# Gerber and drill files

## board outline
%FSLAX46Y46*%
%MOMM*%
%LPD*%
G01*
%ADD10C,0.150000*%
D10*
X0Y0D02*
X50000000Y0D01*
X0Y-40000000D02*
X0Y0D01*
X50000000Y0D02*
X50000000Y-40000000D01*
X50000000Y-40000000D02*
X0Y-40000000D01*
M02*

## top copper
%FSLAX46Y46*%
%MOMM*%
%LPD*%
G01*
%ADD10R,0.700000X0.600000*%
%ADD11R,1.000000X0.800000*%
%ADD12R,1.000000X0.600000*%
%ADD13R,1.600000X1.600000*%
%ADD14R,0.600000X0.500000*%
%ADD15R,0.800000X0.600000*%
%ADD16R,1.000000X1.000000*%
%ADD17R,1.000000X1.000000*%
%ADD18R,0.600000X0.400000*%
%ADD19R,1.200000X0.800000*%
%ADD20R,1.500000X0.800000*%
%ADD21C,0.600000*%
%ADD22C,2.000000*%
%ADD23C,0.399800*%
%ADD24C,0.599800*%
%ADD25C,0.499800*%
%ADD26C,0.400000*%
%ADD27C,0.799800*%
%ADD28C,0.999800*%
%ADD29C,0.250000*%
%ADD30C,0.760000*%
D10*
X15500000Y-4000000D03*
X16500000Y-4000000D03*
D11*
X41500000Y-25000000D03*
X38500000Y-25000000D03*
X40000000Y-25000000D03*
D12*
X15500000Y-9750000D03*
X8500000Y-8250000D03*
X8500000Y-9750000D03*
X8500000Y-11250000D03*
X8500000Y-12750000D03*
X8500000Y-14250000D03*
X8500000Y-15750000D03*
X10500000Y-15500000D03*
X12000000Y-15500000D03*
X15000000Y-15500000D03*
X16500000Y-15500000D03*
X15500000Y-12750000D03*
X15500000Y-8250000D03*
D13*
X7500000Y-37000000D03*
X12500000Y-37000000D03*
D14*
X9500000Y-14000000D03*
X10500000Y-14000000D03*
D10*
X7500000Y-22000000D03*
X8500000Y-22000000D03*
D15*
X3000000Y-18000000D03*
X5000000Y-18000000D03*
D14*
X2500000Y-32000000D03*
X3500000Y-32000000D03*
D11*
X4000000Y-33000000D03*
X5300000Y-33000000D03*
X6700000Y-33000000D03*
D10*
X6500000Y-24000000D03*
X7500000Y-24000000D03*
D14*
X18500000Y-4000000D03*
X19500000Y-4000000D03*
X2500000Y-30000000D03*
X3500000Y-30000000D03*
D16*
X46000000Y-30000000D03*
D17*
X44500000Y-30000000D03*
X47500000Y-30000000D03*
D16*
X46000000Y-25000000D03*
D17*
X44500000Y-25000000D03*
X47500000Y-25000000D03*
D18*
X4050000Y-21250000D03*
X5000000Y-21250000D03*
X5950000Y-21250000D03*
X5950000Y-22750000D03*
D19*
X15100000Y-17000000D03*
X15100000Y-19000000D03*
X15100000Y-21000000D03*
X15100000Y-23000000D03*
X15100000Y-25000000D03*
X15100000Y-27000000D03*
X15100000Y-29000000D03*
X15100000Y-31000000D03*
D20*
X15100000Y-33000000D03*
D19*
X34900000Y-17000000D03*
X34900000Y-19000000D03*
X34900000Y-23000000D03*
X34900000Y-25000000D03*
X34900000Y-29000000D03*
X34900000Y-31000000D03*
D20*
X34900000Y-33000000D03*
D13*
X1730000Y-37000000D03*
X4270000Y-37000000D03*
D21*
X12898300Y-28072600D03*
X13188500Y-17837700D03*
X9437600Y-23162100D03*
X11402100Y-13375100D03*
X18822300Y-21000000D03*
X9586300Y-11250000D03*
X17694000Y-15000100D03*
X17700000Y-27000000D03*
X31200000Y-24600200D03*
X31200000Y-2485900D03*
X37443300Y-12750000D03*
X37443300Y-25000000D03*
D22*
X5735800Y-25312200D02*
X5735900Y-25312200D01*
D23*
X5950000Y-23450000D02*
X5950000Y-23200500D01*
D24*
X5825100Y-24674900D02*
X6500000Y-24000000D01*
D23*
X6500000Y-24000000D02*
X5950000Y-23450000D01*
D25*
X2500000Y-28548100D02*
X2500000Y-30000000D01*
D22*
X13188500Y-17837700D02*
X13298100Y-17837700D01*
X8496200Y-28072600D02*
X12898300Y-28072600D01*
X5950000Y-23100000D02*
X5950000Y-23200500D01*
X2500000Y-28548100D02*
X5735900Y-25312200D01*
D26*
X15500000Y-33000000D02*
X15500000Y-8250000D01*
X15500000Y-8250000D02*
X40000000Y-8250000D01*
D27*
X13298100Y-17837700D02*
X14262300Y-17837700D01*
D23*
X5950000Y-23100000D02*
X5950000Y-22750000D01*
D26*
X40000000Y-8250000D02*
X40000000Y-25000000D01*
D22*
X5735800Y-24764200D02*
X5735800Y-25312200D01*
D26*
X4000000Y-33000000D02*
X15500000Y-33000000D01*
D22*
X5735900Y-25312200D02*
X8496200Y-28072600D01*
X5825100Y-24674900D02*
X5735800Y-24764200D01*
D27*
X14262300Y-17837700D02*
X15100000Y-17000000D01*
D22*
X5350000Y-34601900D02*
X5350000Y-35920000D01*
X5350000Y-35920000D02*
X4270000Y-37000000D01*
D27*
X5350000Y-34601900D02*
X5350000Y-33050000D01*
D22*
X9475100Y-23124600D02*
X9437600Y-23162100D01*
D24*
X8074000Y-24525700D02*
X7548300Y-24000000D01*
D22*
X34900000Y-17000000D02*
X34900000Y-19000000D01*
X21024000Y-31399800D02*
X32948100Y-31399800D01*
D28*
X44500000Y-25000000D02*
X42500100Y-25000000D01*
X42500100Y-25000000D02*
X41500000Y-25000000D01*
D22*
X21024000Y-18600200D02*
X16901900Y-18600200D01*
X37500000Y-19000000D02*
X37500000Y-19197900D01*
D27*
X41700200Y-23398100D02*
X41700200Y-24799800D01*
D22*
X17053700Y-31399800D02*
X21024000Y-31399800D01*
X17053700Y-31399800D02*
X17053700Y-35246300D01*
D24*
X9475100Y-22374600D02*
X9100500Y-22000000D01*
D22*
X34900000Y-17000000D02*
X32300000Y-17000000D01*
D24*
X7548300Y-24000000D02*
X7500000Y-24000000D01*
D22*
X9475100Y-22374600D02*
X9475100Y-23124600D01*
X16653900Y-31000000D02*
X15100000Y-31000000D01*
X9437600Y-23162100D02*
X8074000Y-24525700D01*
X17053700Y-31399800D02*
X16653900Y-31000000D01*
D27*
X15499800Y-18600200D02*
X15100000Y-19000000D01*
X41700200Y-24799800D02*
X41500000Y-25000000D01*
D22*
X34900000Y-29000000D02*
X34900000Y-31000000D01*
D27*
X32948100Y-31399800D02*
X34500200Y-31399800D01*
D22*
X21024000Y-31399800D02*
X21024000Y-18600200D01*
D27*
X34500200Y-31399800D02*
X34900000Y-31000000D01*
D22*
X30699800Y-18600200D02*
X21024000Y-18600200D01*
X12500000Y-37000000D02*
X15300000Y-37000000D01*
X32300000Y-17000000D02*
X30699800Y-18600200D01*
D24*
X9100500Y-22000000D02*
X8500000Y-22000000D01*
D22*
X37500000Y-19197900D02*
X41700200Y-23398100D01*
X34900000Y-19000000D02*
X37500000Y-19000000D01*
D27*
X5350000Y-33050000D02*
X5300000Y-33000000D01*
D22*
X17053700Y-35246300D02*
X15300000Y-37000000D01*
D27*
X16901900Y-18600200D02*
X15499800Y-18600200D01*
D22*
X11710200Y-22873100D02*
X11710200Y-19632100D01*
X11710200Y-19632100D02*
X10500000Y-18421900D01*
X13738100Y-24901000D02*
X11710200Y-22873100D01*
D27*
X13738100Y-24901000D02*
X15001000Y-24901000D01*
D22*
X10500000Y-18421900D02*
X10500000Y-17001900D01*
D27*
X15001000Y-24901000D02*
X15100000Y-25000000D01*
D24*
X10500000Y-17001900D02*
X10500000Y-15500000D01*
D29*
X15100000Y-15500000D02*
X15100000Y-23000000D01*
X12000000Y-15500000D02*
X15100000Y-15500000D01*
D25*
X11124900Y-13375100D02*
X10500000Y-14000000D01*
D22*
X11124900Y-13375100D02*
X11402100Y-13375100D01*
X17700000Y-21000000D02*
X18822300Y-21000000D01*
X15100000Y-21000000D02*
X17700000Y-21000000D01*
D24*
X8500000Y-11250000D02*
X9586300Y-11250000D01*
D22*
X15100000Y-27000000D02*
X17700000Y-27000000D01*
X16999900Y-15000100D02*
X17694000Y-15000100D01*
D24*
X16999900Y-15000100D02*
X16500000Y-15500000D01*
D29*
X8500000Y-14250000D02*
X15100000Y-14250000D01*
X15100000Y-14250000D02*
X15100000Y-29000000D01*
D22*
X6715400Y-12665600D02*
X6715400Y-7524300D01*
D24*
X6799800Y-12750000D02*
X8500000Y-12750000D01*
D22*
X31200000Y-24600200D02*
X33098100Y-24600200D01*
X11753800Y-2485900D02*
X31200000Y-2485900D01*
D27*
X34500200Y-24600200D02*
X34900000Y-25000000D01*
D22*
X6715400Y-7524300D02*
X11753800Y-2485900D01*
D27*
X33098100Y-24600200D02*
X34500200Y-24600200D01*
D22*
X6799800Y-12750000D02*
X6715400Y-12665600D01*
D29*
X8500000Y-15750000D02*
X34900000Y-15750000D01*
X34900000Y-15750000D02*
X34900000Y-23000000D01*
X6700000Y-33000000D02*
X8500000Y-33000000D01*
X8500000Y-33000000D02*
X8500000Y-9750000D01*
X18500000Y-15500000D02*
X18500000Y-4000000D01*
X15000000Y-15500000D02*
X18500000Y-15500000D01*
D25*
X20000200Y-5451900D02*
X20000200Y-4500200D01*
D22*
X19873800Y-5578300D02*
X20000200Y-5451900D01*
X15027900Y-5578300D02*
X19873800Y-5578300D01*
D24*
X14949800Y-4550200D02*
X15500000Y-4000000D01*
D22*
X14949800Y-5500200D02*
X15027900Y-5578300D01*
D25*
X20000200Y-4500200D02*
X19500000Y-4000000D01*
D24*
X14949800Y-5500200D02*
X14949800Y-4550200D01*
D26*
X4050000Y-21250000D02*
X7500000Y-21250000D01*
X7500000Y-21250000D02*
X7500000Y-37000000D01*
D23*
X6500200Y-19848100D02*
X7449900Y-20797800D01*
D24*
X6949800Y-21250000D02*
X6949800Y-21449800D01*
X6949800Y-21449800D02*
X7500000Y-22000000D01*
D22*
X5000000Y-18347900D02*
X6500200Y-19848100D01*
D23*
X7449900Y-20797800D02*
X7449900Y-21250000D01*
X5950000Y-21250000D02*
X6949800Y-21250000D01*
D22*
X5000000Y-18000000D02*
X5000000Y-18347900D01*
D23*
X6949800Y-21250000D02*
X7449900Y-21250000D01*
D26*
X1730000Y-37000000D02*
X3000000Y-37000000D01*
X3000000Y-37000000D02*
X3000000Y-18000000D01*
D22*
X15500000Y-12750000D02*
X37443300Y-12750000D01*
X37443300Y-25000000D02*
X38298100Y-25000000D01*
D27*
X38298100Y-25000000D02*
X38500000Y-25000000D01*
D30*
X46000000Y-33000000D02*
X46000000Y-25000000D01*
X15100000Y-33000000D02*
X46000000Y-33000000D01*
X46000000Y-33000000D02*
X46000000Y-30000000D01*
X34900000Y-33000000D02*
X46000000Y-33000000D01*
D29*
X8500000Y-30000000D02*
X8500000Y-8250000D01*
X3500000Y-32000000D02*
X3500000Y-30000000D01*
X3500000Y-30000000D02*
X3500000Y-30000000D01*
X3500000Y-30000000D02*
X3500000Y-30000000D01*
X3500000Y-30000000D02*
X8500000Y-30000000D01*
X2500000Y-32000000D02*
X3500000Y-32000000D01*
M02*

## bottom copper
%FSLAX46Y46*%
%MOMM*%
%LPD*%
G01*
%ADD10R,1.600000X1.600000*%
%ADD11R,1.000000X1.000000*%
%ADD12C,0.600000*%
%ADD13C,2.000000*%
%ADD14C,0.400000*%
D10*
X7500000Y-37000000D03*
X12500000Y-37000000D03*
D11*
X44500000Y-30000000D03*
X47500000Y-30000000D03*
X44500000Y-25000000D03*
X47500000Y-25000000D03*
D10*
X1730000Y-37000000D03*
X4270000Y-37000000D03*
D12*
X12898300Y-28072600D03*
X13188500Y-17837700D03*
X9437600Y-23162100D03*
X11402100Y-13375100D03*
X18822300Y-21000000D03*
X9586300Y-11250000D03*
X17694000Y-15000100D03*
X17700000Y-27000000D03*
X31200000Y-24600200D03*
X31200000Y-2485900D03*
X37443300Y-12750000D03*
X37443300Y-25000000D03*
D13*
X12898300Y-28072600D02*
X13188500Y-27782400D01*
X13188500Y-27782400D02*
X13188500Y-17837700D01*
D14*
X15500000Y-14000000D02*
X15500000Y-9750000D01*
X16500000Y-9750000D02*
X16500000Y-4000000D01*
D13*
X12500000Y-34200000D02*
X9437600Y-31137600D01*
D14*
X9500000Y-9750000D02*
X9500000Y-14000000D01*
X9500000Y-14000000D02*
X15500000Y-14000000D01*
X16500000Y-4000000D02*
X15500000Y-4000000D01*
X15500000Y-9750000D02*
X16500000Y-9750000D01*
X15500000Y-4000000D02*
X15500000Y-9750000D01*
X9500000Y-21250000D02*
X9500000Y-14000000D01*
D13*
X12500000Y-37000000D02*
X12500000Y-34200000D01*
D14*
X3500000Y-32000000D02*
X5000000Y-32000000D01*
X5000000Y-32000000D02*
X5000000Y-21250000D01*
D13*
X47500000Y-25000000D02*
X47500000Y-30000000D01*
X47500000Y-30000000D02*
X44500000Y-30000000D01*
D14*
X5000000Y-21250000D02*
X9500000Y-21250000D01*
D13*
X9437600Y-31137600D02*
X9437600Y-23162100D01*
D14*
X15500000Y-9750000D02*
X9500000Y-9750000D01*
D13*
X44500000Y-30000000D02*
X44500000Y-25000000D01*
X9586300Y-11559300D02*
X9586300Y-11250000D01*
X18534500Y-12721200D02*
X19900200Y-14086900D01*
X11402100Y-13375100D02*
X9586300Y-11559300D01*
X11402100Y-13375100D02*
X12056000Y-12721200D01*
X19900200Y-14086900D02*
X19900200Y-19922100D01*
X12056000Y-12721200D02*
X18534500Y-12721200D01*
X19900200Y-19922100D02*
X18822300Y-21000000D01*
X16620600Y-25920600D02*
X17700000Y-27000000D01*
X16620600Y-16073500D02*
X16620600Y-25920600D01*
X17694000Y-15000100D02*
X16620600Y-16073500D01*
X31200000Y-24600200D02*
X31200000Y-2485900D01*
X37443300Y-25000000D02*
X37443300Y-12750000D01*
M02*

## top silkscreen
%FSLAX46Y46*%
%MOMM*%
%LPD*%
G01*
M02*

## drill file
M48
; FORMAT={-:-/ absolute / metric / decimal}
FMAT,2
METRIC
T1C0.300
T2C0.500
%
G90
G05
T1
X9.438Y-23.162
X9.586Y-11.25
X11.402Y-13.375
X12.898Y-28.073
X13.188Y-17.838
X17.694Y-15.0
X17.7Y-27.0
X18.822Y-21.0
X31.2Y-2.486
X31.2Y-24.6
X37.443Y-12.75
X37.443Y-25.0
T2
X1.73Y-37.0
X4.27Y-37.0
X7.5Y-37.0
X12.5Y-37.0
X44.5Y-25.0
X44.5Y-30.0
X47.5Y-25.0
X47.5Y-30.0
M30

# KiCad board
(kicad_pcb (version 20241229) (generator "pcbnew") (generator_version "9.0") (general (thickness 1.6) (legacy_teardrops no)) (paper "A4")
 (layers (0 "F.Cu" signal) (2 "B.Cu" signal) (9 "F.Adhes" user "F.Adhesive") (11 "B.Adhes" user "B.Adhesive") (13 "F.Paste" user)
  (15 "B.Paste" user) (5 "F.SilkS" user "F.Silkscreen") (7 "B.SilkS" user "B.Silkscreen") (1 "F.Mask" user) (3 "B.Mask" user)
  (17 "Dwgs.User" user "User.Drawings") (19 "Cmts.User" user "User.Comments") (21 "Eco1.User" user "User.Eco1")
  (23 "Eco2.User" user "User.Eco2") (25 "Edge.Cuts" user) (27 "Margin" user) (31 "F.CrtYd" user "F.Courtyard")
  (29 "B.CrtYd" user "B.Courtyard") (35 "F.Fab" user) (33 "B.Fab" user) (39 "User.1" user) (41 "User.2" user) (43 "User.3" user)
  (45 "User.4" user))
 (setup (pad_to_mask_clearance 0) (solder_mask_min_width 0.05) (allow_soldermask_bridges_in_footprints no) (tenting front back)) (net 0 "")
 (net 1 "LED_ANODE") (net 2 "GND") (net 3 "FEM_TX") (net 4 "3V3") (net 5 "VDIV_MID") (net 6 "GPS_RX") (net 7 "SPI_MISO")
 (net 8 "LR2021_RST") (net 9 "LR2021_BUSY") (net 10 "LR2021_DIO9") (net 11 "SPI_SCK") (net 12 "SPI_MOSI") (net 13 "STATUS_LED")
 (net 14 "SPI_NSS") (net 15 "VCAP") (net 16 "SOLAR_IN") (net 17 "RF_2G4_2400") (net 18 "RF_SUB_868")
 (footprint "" (layer "F.Cu") (at 16 4)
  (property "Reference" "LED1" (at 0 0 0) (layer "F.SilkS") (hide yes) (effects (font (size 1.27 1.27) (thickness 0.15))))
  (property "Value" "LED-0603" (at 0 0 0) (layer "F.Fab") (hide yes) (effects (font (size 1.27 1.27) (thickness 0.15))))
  (pad "A" smd rect (at -0.5 0) (size 0.7 0.6) (layers "F.Cu" "F.Mask") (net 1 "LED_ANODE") (thermal_bridge_angle 45))
  (pad "K" smd rect (at 0.5 0) (size 0.7 0.6) (layers "F.Cu" "F.Mask") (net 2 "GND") (thermal_bridge_angle 45)))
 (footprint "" (layer "F.Cu") (at 40 25)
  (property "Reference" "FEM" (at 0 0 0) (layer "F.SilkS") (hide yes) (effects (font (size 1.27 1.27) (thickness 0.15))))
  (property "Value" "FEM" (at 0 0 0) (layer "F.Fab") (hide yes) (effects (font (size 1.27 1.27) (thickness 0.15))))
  (pad "GND" smd rect (at 1.5 0) (size 1 0.8) (layers "F.Cu" "F.Mask") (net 2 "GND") (thermal_bridge_angle 45))
  (pad "TX" smd rect (at -1.5 0) (size 1 0.8) (layers "F.Cu" "F.Mask") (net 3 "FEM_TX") (thermal_bridge_angle 45))
  (pad "VCC" smd rect (at 0 0) (size 1 0.8) (layers "F.Cu" "F.Mask") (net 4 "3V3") (thermal_bridge_angle 45)))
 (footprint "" (layer "F.Cu") (at 12 12)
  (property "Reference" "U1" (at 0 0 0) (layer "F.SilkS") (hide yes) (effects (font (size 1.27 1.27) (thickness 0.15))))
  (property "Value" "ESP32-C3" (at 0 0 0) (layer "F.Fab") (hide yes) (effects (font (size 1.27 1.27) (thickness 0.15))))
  (pad "GND" smd rect (at 3.5 -2.25) (size 1 0.6) (layers "F.Cu" "F.Mask") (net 2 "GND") (thermal_bridge_angle 45))
  (pad "GPIO0" smd rect (at -3.5 -3.75) (size 1 0.6) (layers "F.Cu" "F.Mask") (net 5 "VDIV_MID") (thermal_bridge_angle 45))
  (pad "GPIO1" smd rect (at -3.5 -2.25) (size 1 0.6) (layers "F.Cu" "F.Mask") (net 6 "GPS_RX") (thermal_bridge_angle 45))
  (pad "GPIO2" smd rect (at -3.5 -0.75) (size 1 0.6) (layers "F.Cu" "F.Mask") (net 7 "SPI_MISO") (thermal_bridge_angle 45))
  (pad "GPIO3" smd rect (at -3.5 0.75) (size 1 0.6) (layers "F.Cu" "F.Mask") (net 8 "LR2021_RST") (thermal_bridge_angle 45))
  (pad "GPIO4" smd rect (at -3.5 2.25) (size 1 0.6) (layers "F.Cu" "F.Mask") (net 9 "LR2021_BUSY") (thermal_bridge_angle 45))
  (pad "GPIO5" smd rect (at -3.5 3.75) (size 1 0.6) (layers "F.Cu" "F.Mask") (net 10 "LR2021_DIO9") (thermal_bridge_angle 45))
  (pad "GPIO6" smd rect (at -1.5 3.5) (size 1 0.6) (layers "F.Cu" "F.Mask") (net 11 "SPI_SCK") (thermal_bridge_angle 45))
  (pad "GPIO7" smd rect (at 0 3.5) (size 1 0.6) (layers "F.Cu" "F.Mask") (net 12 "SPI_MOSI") (thermal_bridge_angle 45))
  (pad "GPIO9" smd rect (at 3 3.5) (size 1 0.6) (layers "F.Cu" "F.Mask") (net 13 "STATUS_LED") (thermal_bridge_angle 45))
  (pad "GPIO10" smd rect (at 4.5 3.5) (size 1 0.6) (layers "F.Cu" "F.Mask") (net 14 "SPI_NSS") (thermal_bridge_angle 45))
  (pad "GPIO19" smd rect (at 3.5 0.75) (size 1 0.6) (layers "F.Cu" "F.Mask") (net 3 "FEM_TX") (thermal_bridge_angle 45))
  (pad "VCC" smd rect (at 3.5 -3.75) (size 1 0.6) (layers "F.Cu" "F.Mask") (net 4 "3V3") (thermal_bridge_angle 45)))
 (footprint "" (layer "F.Cu") (at 10 37)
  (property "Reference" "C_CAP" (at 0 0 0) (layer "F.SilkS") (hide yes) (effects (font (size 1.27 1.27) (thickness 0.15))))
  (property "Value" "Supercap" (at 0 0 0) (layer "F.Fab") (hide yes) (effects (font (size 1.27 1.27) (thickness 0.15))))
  (pad "1" thru_hole rect (at -2.5 0) (size 1.6 1.6) (drill 0.5) (layers "*.Cu" "*.Mask") (remove_unused_layers no) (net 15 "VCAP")
   (thermal_bridge_angle 45))
  (pad "2" thru_hole rect (at 2.5 0) (size 1.6 1.6) (drill 0.5) (layers "*.Cu" "*.Mask") (remove_unused_layers no) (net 2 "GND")
   (thermal_bridge_angle 45)))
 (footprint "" (layer "F.Cu") (at 10 14)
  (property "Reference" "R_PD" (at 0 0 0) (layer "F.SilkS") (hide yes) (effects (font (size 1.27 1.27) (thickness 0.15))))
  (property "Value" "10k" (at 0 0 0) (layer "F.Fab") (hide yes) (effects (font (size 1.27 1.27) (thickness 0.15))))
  (pad "1" smd rect (at -0.5 0) (size 0.6 0.5) (layers "F.Cu" "F.Mask") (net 2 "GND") (thermal_bridge_angle 45))
  (pad "2" smd rect (at 0.5 0) (size 0.6 0.5) (layers "F.Cu" "F.Mask") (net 7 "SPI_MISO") (thermal_bridge_angle 45)))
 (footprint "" (layer "F.Cu") (at 8 22)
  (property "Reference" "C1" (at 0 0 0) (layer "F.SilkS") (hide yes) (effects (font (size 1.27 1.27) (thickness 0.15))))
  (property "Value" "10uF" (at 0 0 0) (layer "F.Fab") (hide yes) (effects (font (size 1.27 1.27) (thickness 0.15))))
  (pad "1" smd rect (at -0.5 0) (size 0.7 0.6) (layers "F.Cu" "F.Mask") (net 15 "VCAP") (thermal_bridge_angle 45))
  (pad "2" smd rect (at 0.5 0) (size 0.7 0.6) (layers "F.Cu" "F.Mask") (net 2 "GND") (thermal_bridge_angle 45)))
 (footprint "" (layer "F.Cu") (at 4 18)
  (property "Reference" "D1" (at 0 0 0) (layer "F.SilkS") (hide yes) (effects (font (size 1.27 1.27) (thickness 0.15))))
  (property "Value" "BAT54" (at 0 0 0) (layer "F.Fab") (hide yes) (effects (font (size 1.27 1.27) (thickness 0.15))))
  (pad "A" smd rect (at -1 0) (size 0.8 0.6) (layers "F.Cu" "F.Mask") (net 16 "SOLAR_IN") (thermal_bridge_angle 45))
  (pad "K" smd rect (at 1 0) (size 0.8 0.6) (layers "F.Cu" "F.Mask") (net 15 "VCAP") (thermal_bridge_angle 45)))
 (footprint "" (layer "F.Cu") (at 3 32)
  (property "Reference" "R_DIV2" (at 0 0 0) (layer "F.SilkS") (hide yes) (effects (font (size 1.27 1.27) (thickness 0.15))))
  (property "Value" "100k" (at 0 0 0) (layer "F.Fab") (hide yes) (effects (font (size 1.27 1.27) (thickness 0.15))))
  (pad "1" smd rect (at -0.5 0) (size 0.6 0.5) (layers "F.Cu" "F.Mask") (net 5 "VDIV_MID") (thermal_bridge_angle 45))
  (pad "2" smd rect (at 0.5 0) (size 0.6 0.5) (layers "F.Cu" "F.Mask") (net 2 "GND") (thermal_bridge_angle 45)))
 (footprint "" (layer "F.Cu") (at 6 33)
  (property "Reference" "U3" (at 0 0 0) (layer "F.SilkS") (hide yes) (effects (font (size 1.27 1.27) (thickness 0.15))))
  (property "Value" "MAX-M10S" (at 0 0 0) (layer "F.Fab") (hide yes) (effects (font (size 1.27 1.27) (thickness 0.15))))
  (pad "1" smd rect (at -2 0) (size 1 0.8) (layers "F.Cu" "F.Mask") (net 4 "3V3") (thermal_bridge_angle 45))
  (pad "2" smd rect (at -0.7 0) (size 1 0.8) (layers "F.Cu" "F.Mask") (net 2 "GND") (thermal_bridge_angle 45))
  (pad "3" smd rect (at 0.7 0) (size 1 0.8) (layers "F.Cu" "F.Mask") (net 6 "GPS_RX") (thermal_bridge_angle 45)))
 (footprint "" (layer "F.Cu") (at 7 24)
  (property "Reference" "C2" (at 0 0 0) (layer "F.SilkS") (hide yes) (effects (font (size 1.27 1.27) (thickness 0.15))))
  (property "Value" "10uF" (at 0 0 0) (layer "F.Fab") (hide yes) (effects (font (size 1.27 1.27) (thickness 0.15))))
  (pad "1" smd rect (at -0.5 0) (size 0.7 0.6) (layers "F.Cu" "F.Mask") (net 4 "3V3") (thermal_bridge_angle 45))
  (pad "2" smd rect (at 0.5 0) (size 0.7 0.6) (layers "F.Cu" "F.Mask") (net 2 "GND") (thermal_bridge_angle 45)))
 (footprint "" (layer "F.Cu") (at 19 4)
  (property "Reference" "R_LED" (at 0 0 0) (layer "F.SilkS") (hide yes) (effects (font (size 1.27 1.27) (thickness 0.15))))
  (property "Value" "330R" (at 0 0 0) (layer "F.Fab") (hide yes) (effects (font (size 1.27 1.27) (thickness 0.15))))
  (pad "1" smd rect (at -0.5 0) (size 0.6 0.5) (layers "F.Cu" "F.Mask") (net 13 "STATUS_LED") (thermal_bridge_angle 45))
  (pad "2" smd rect (at 0.5 0) (size 0.6 0.5) (layers "F.Cu" "F.Mask") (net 1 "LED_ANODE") (thermal_bridge_angle 45)))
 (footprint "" (layer "F.Cu") (at 3 30)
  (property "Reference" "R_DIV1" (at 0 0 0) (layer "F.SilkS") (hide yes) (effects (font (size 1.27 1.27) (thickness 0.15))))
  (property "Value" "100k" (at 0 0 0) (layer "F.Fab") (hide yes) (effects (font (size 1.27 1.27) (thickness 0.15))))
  (pad "1" smd rect (at -0.5 0) (size 0.6 0.5) (layers "F.Cu" "F.Mask") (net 4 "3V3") (thermal_bridge_angle 45))
  (pad "2" smd rect (at 0.5 0) (size 0.6 0.5) (layers "F.Cu" "F.Mask") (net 5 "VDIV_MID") (thermal_bridge_angle 45)))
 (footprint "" (layer "F.Cu") (at 46 30)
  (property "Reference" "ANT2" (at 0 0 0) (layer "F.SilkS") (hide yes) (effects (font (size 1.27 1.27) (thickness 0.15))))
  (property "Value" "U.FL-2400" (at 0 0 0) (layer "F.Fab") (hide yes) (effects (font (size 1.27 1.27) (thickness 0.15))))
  (pad "1" smd rect (at 0 0) (size 1 1) (layers "F.Cu" "F.Mask") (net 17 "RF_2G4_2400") (thermal_bridge_angle 45))
  (pad "2" thru_hole rect (at -1.5 0) (size 1 1) (drill 0.5) (layers "*.Cu" "*.Mask") (remove_unused_layers no) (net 2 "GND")
   (thermal_bridge_angle 45))
  (pad "3" thru_hole rect (at 1.5 0) (size 1 1) (drill 0.5) (layers "*.Cu" "*.Mask") (remove_unused_layers no) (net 2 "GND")
   (thermal_bridge_angle 45)))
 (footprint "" (layer "F.Cu") (at 46 25)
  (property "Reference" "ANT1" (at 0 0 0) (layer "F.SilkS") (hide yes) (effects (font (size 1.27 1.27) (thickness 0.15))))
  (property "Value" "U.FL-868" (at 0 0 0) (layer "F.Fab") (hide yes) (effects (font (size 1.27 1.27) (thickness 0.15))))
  (pad "1" smd rect (at 0 0) (size 1 1) (layers "F.Cu" "F.Mask") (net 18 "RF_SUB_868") (thermal_bridge_angle 45))
  (pad "2" thru_hole rect (at -1.5 0) (size 1 1) (drill 0.5) (layers "*.Cu" "*.Mask") (remove_unused_layers no) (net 2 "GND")
   (thermal_bridge_angle 45))
  (pad "3" thru_hole rect (at 1.5 0) (size 1 1) (drill 0.5) (layers "*.Cu" "*.Mask") (remove_unused_layers no) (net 2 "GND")
   (thermal_bridge_angle 45)))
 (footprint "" (layer "F.Cu") (at 5 22)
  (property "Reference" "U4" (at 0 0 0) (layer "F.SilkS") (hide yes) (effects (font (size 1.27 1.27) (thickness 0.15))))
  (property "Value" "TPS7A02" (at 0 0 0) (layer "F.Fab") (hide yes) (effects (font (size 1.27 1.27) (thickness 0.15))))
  (pad "1" smd rect (at -0.95 -0.75) (size 0.6 0.4) (layers "F.Cu" "F.Mask") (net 15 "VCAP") (thermal_bridge_angle 45))
  (pad "2" smd rect (at 0 -0.75) (size 0.6 0.4) (layers "F.Cu" "F.Mask") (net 2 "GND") (thermal_bridge_angle 45))
  (pad "3" smd rect (at 0.95 -0.75) (size 0.6 0.4) (layers "F.Cu" "F.Mask") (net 15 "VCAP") (thermal_bridge_angle 45))
  (pad "4" smd rect (at 0.95 0.75) (size 0.6 0.4) (layers "F.Cu" "F.Mask") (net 4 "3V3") (thermal_bridge_angle 45)))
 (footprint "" (layer "F.Cu") (at 25 25)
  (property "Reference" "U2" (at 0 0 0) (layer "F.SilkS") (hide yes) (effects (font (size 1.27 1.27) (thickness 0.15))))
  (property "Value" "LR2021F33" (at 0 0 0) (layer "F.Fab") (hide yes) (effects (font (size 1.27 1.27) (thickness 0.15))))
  (pad "1" smd rect (at -9.9 -8) (size 1.2 0.8) (layers "F.Cu" "F.Mask") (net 4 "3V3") (thermal_bridge_angle 45))
  (pad "2" smd rect (at -9.9 -6) (size 1.2 0.8) (layers "F.Cu" "F.Mask") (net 2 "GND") (thermal_bridge_angle 45))
  (pad "3" smd rect (at -9.9 -4) (size 1.2 0.8) (layers "F.Cu" "F.Mask") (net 7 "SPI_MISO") (thermal_bridge_angle 45))
  (pad "4" smd rect (at -9.9 -2) (size 1.2 0.8) (layers "F.Cu" "F.Mask") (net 12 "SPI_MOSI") (thermal_bridge_angle 45))
  (pad "5" smd rect (at -9.9 0) (size 1.2 0.8) (layers "F.Cu" "F.Mask") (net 11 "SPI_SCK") (thermal_bridge_angle 45))
  (pad "6" smd rect (at -9.9 2) (size 1.2 0.8) (layers "F.Cu" "F.Mask") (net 14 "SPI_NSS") (thermal_bridge_angle 45))
  (pad "7" smd rect (at -9.9 4) (size 1.2 0.8) (layers "F.Cu" "F.Mask") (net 9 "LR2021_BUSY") (thermal_bridge_angle 45))
  (pad "8" smd rect (at -9.9 6) (size 1.2 0.8) (layers "F.Cu" "F.Mask") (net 2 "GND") (thermal_bridge_angle 45))
  (pad "9" smd rect (at -9.9 8) (size 1.5 0.8) (layers "F.Cu" "F.Mask") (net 18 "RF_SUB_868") (thermal_bridge_angle 45))
  (pad "10" smd rect (at 9.9 -8) (size 1.2 0.8) (layers "F.Cu" "F.Mask") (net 2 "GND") (thermal_bridge_angle 45))
  (pad "11" smd rect (at 9.9 -6) (size 1.2 0.8) (layers "F.Cu" "F.Mask") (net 2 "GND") (thermal_bridge_angle 45))
  (pad "13" smd rect (at 9.9 -2) (size 1.2 0.8) (layers "F.Cu" "F.Mask") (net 10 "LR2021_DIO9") (thermal_bridge_angle 45))
  (pad "14" smd rect (at 9.9 0) (size 1.2 0.8) (layers "F.Cu" "F.Mask") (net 8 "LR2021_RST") (thermal_bridge_angle 45))
  (pad "16" smd rect (at 9.9 4) (size 1.2 0.8) (layers "F.Cu" "F.Mask") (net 2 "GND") (thermal_bridge_angle 45))
  (pad "17" smd rect (at 9.9 6) (size 1.2 0.8) (layers "F.Cu" "F.Mask") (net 2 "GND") (thermal_bridge_angle 45))
  (pad "18" smd rect (at 9.9 8) (size 1.5 0.8) (layers "F.Cu" "F.Mask") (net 17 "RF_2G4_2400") (thermal_bridge_angle 45)))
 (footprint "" (layer "F.Cu") (at 3 37)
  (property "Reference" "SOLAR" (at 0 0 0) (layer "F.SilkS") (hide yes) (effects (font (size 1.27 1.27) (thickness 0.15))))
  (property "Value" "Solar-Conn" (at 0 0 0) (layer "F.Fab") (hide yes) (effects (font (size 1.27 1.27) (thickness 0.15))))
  (pad "1" thru_hole rect (at -1.27 0) (size 1.6 1.6) (drill 0.5) (layers "*.Cu" "*.Mask") (remove_unused_layers no) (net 16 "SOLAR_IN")
   (thermal_bridge_angle 45))
  (pad "2" thru_hole rect (at 1.27 0) (size 1.6 1.6) (drill 0.5) (layers "*.Cu" "*.Mask") (remove_unused_layers no) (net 2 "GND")
   (thermal_bridge_angle 45)))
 (gr_line (start 0 0) (end 50 0) (stroke (width 0.15) (type default)) (layer "Edge.Cuts"))
 (gr_line (start 0 40) (end 0 0) (stroke (width 0.15) (type default)) (layer "Edge.Cuts"))
 (gr_line (start 50 0) (end 50 40) (stroke (width 0.15) (type default)) (layer "Edge.Cuts"))
 (gr_line (start 50 40) (end 0 40) (stroke (width 0.15) (type default)) (layer "Edge.Cuts"))
 (segment (start 5.7358 25.3122) (end 5.7359 25.3122) (width 2) (layer "F.Cu") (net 4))
 (segment (start 5.95 23.45) (end 5.95 23.2005) (width 0.3998) (layer "F.Cu") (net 4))
 (segment (start 5.8251 24.6749) (end 6.5 24) (width 0.5998) (layer "F.Cu") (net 4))
 (segment (start 6.5 24) (end 5.95 23.45) (width 0.3998) (layer "F.Cu") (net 4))
 (segment (start 2.5 28.5481) (end 2.5 30) (width 0.4998) (layer "F.Cu") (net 4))
 (segment (start 13.1885 17.8377) (end 13.2981 17.8377) (width 2) (layer "F.Cu") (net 4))
 (segment (start 8.4962 28.0726) (end 12.8983 28.0726) (width 2) (layer "F.Cu") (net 4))
 (segment (start 5.95 23.1) (end 5.95 23.2005) (width 2) (layer "F.Cu") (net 4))
 (segment (start 2.5 28.5481) (end 5.7359 25.3122) (width 2) (layer "F.Cu") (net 4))
 (segment (start 15.5 33) (end 15.5 8.25) (width 0.4) (layer "F.Cu") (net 4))
 (segment (start 15.5 8.25) (end 40 8.25) (width 0.4) (layer "F.Cu") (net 4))
 (segment (start 13.2981 17.8377) (end 14.2623 17.8377) (width 0.7998) (layer "F.Cu") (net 4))
 (segment (start 5.95 23.1) (end 5.95 22.75) (width 0.3998) (layer "F.Cu") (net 4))
 (segment (start 40 8.25) (end 40 25) (width 0.4) (layer "F.Cu") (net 4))
 (segment (start 5.7358 24.7642) (end 5.7358 25.3122) (width 2) (layer "F.Cu") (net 4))
 (segment (start 4 33) (end 15.5 33) (width 0.4) (layer "F.Cu") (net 4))
 (segment (start 5.7359 25.3122) (end 8.4962 28.0726) (width 2) (layer "F.Cu") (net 4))
 (segment (start 5.8251 24.6749) (end 5.7358 24.7642) (width 2) (layer "F.Cu") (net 4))
 (segment (start 14.2623 17.8377) (end 15.1 17) (width 0.7998) (layer "F.Cu") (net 4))
 (via (at 12.8983 28.0726) (size 0.6) (drill 0.3) (layers "F.Cu" "B.Cu") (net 4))
 (via (at 13.1885 17.8377) (size 0.6) (drill 0.3) (layers "F.Cu" "B.Cu") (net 4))
 (segment (start 12.8983 28.0726) (end 13.1885 27.7824) (width 2) (layer "B.Cu") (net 4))
 (segment (start 13.1885 27.7824) (end 13.1885 17.8377) (width 2) (layer "B.Cu") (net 4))
 (segment (start 5.35 34.6019) (end 5.35 35.92) (width 2) (layer "F.Cu") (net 2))
 (segment (start 5.35 35.92) (end 4.27 37) (width 2) (layer "F.Cu") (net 2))
 (segment (start 5.35 34.6019) (end 5.35 33.05) (width 0.7998) (layer "F.Cu") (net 2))
 (segment (start 9.4751 23.1246) (end 9.4376 23.1621) (width 2) (layer "F.Cu") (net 2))
 (segment (start 8.074 24.5257) (end 7.5483 24) (width 0.5998) (layer "F.Cu") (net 2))
 (segment (start 34.9 17) (end 34.9 19) (width 2) (layer "F.Cu") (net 2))
 (segment (start 21.024 31.3998) (end 32.9481 31.3998) (width 2) (layer "F.Cu") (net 2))
 (segment (start 44.5 25) (end 42.5001 25) (width 0.9998) (layer "F.Cu") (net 2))
 (segment (start 42.5001 25) (end 41.5 25) (width 0.9998) (layer "F.Cu") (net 2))
 (segment (start 21.024 18.6002) (end 16.9019 18.6002) (width 2) (layer "F.Cu") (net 2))
 (segment (start 37.5 19) (end 37.5 19.1979) (width 2) (layer "F.Cu") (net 2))
 (segment (start 41.7002 23.3981) (end 41.7002 24.7998) (width 0.7998) (layer "F.Cu") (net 2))
 (segment (start 17.0537 31.3998) (end 21.024 31.3998) (width 2) (layer "F.Cu") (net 2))
 (segment (start 17.0537 31.3998) (end 17.0537 35.2463) (width 2) (layer "F.Cu") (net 2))
 (segment (start 9.4751 22.3746) (end 9.1005 22) (width 0.5998) (layer "F.Cu") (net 2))
 (segment (start 34.9 17) (end 32.3 17) (width 2) (layer "F.Cu") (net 2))
 (segment (start 7.5483 24) (end 7.5 24) (width 0.5998) (layer "F.Cu") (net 2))
 (segment (start 9.4751 22.3746) (end 9.4751 23.1246) (width 2) (layer "F.Cu") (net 2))
 (segment (start 16.6539 31) (end 15.1 31) (width 2) (layer "F.Cu") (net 2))
 (segment (start 9.4376 23.1621) (end 8.074 24.5257) (width 2) (layer "F.Cu") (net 2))
 (segment (start 17.0537 31.3998) (end 16.6539 31) (width 2) (layer "F.Cu") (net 2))
 (segment (start 15.4998 18.6002) (end 15.1 19) (width 0.7998) (layer "F.Cu") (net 2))
 (segment (start 41.7002 24.7998) (end 41.5 25) (width 0.7998) (layer "F.Cu") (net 2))
 (segment (start 34.9 29) (end 34.9 31) (width 2) (layer "F.Cu") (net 2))
 (segment (start 32.9481 31.3998) (end 34.5002 31.3998) (width 0.7998) (layer "F.Cu") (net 2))
 (segment (start 21.024 31.3998) (end 21.024 18.6002) (width 2) (layer "F.Cu") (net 2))
 (segment (start 34.5002 31.3998) (end 34.9 31) (width 0.7998) (layer "F.Cu") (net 2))
 (segment (start 30.6998 18.6002) (end 21.024 18.6002) (width 2) (layer "F.Cu") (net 2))
 (segment (start 12.5 37) (end 15.3 37) (width 2) (layer "F.Cu") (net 2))
 (segment (start 32.3 17) (end 30.6998 18.6002) (width 2) (layer "F.Cu") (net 2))
 (segment (start 9.1005 22) (end 8.5 22) (width 0.5998) (layer "F.Cu") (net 2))
 (segment (start 37.5 19.1979) (end 41.7002 23.3981) (width 2) (layer "F.Cu") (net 2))
 (segment (start 34.9 19) (end 37.5 19) (width 2) (layer "F.Cu") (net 2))
 (segment (start 5.35 33.05) (end 5.3 33) (width 0.7998) (layer "F.Cu") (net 2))
 (segment (start 17.0537 35.2463) (end 15.3 37) (width 2) (layer "F.Cu") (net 2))
 (segment (start 16.9019 18.6002) (end 15.4998 18.6002) (width 0.7998) (layer "F.Cu") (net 2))
 (via (at 9.4376 23.1621) (size 0.6) (drill 0.3) (layers "F.Cu" "B.Cu") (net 2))
 (segment (start 15.5 14) (end 15.5 9.75) (width 0.4) (layer "B.Cu") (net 2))
 (segment (start 16.5 9.75) (end 16.5 4) (width 0.4) (layer "B.Cu") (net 2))
 (segment (start 12.5 34.2) (end 9.4376 31.1376) (width 2) (layer "B.Cu") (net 2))
 (segment (start 9.5 9.75) (end 9.5 14) (width 0.4) (layer "B.Cu") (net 2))
 (segment (start 9.5 14) (end 15.5 14) (width 0.4) (layer "B.Cu") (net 2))
 (segment (start 16.5 4) (end 15.5 4) (width 0.4) (layer "B.Cu") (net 2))
 (segment (start 15.5 9.75) (end 16.5 9.75) (width 0.4) (layer "B.Cu") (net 2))
 (segment (start 15.5 4) (end 15.5 9.75) (width 0.4) (layer "B.Cu") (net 2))
 (segment (start 9.5 21.25) (end 9.5 14) (width 0.4) (layer "B.Cu") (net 2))
 (segment (start 12.5 37) (end 12.5 34.2) (width 2) (layer "B.Cu") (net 2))
 (segment (start 3.5 32) (end 5 32) (width 0.4) (layer "B.Cu") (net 2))
 (segment (start 5 32) (end 5 21.25) (width 0.4) (layer "B.Cu") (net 2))
 (segment (start 47.5 25) (end 47.5 30) (width 2) (layer "B.Cu") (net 2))
 (segment (start 47.5 30) (end 44.5 30) (width 2) (layer "B.Cu") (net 2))
 (segment (start 5 21.25) (end 9.5 21.25) (width 0.4) (layer "B.Cu") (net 2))
 (segment (start 9.4376 31.1376) (end 9.4376 23.1621) (width 2) (layer "B.Cu") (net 2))
 (segment (start 15.5 9.75) (end 9.5 9.75) (width 0.4) (layer "B.Cu") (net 2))
 (segment (start 44.5 30) (end 44.5 25) (width 2) (layer "B.Cu") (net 2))
 (segment (start 11.7102 22.8731) (end 11.7102 19.6321) (width 2) (layer "F.Cu") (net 11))
 (segment (start 11.7102 19.6321) (end 10.5 18.4219) (width 2) (layer "F.Cu") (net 11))
 (segment (start 13.7381 24.901) (end 11.7102 22.8731) (width 2) (layer "F.Cu") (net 11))
 (segment (start 13.7381 24.901) (end 15.001 24.901) (width 0.7998) (layer "F.Cu") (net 11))
 (segment (start 10.5 18.4219) (end 10.5 17.0019) (width 2) (layer "F.Cu") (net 11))
 (segment (start 15.001 24.901) (end 15.1 25) (width 0.7998) (layer "F.Cu") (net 11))
 (segment (start 10.5 17.0019) (end 10.5 15.5) (width 0.5998) (layer "F.Cu") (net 11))
 (segment (start 15.1 15.5) (end 15.1 23) (width 0.25) (layer "F.Cu") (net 12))
 (segment (start 12 15.5) (end 15.1 15.5) (width 0.25) (layer "F.Cu") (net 12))
 (segment (start 11.1249 13.3751) (end 10.5 14) (width 0.4998) (layer "F.Cu") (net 7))
 (segment (start 11.1249 13.3751) (end 11.4021 13.3751) (width 2) (layer "F.Cu") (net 7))
 (segment (start 17.7 21) (end 18.8223 21) (width 2) (layer "F.Cu") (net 7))
 (segment (start 15.1 21) (end 17.7 21) (width 2) (layer "F.Cu") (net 7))
 (segment (start 8.5 11.25) (end 9.5863 11.25) (width 0.5998) (layer "F.Cu") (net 7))
 (via (at 11.4021 13.3751) (size 0.6) (drill 0.3) (layers "F.Cu" "B.Cu") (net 7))
 (via (at 18.8223 21) (size 0.6) (drill 0.3) (layers "F.Cu" "B.Cu") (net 7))
 (via (at 9.5863 11.25) (size 0.6) (drill 0.3) (layers "F.Cu" "B.Cu") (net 7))
 (segment (start 9.5863 11.5593) (end 9.5863 11.25) (width 2) (layer "B.Cu") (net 7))
 (segment (start 18.5345 12.7212) (end 19.9002 14.0869) (width 2) (layer "B.Cu") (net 7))
 (segment (start 11.4021 13.3751) (end 9.5863 11.5593) (width 2) (layer "B.Cu") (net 7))
 (segment (start 11.4021 13.3751) (end 12.056 12.7212) (width 2) (layer "B.Cu") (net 7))
 (segment (start 19.9002 14.0869) (end 19.9002 19.9221) (width 2) (layer "B.Cu") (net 7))
 (segment (start 12.056 12.7212) (end 18.5345 12.7212) (width 2) (layer "B.Cu") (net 7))
 (segment (start 19.9002 19.9221) (end 18.8223 21) (width 2) (layer "B.Cu") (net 7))
 (segment (start 15.1 27) (end 17.7 27) (width 2) (layer "F.Cu") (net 14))
 (segment (start 16.9999 15.0001) (end 17.694 15.0001) (width 2) (layer "F.Cu") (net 14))
 (segment (start 16.9999 15.0001) (end 16.5 15.5) (width 0.5998) (layer "F.Cu") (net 14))
 (via (at 17.694 15.0001) (size 0.6) (drill 0.3) (layers "F.Cu" "B.Cu") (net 14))
 (via (at 17.7 27) (size 0.6) (drill 0.3) (layers "F.Cu" "B.Cu") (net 14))
 (segment (start 16.6206 25.9206) (end 17.7 27) (width 2) (layer "B.Cu") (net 14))
 (segment (start 16.6206 16.0735) (end 16.6206 25.9206) (width 2) (layer "B.Cu") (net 14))
 (segment (start 17.694 15.0001) (end 16.6206 16.0735) (width 2) (layer "B.Cu") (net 14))
 (segment (start 8.5 14.25) (end 15.1 14.25) (width 0.25) (layer "F.Cu") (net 9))
 (segment (start 15.1 14.25) (end 15.1 29) (width 0.25) (layer "F.Cu") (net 9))
 (segment (start 6.7154 12.6656) (end 6.7154 7.5243) (width 2) (layer "F.Cu") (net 8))
 (segment (start 6.7998 12.75) (end 8.5 12.75) (width 0.5998) (layer "F.Cu") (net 8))
 (segment (start 31.2 24.6002) (end 33.0981 24.6002) (width 2) (layer "F.Cu") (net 8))
 (segment (start 11.7538 2.4859) (end 31.2 2.4859) (width 2) (layer "F.Cu") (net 8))
 (segment (start 34.5002 24.6002) (end 34.9 25) (width 0.7998) (layer "F.Cu") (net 8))
 (segment (start 6.7154 7.5243) (end 11.7538 2.4859) (width 2) (layer "F.Cu") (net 8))
 (segment (start 33.0981 24.6002) (end 34.5002 24.6002) (width 0.7998) (layer "F.Cu") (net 8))
 (segment (start 6.7998 12.75) (end 6.7154 12.6656) (width 2) (layer "F.Cu") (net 8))
 (via (at 31.2 24.6002) (size 0.6) (drill 0.3) (layers "F.Cu" "B.Cu") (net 8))
 (via (at 31.2 2.4859) (size 0.6) (drill 0.3) (layers "F.Cu" "B.Cu") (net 8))
 (segment (start 31.2 24.6002) (end 31.2 2.4859) (width 2) (layer "B.Cu") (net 8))
 (segment (start 8.5 15.75) (end 34.9 15.75) (width 0.25) (layer "F.Cu") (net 10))
 (segment (start 34.9 15.75) (end 34.9 23) (width 0.25) (layer "F.Cu") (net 10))
 (segment (start 6.7 33) (end 8.5 33) (width 0.25) (layer "F.Cu") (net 6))
 (segment (start 8.5 33) (end 8.5 9.75) (width 0.25) (layer "F.Cu") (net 6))
 (segment (start 18.5 15.5) (end 18.5 4) (width 0.25) (layer "F.Cu") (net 13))
 (segment (start 15 15.5) (end 18.5 15.5) (width 0.25) (layer "F.Cu") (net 13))
 (segment (start 20.0002 5.4519) (end 20.0002 4.5002) (width 0.4998) (layer "F.Cu") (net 1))
 (segment (start 19.8738 5.5783) (end 20.0002 5.4519) (width 2) (layer "F.Cu") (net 1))
 (segment (start 15.0279 5.5783) (end 19.8738 5.5783) (width 2) (layer "F.Cu") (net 1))
 (segment (start 14.9498 4.5502) (end 15.5 4) (width 0.5998) (layer "F.Cu") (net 1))
 (segment (start 14.9498 5.5002) (end 15.0279 5.5783) (width 2) (layer "F.Cu") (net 1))
 (segment (start 20.0002 4.5002) (end 19.5 4) (width 0.4998) (layer "F.Cu") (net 1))
 (segment (start 14.9498 5.5002) (end 14.9498 4.5502) (width 0.5998) (layer "F.Cu") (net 1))
 (segment (start 4.05 21.25) (end 7.5 21.25) (width 0.4) (layer "F.Cu") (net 15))
 (segment (start 7.5 21.25) (end 7.5 37) (width 0.4) (layer "F.Cu") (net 15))
 (segment (start 6.5002 19.8481) (end 7.4499 20.7978) (width 0.3998) (layer "F.Cu") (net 15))
 (segment (start 6.9498 21.25) (end 6.9498 21.4498) (width 0.5998) (layer "F.Cu") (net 15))
 (segment (start 6.9498 21.4498) (end 7.5 22) (width 0.5998) (layer "F.Cu") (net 15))
 (segment (start 5 18.3479) (end 6.5002 19.8481) (width 2) (layer "F.Cu") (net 15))
 (segment (start 7.4499 20.7978) (end 7.4499 21.25) (width 0.3998) (layer "F.Cu") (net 15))
 (segment (start 5.95 21.25) (end 6.9498 21.25) (width 0.3998) (layer "F.Cu") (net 15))
 (segment (start 5 18) (end 5 18.3479) (width 2) (layer "F.Cu") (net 15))
 (segment (start 6.9498 21.25) (end 7.4499 21.25) (width 0.3998) (layer "F.Cu") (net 15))
 (segment (start 1.73 37) (end 3 37) (width 0.4) (layer "F.Cu") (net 16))
 (segment (start 3 37) (end 3 18) (width 0.4) (layer "F.Cu") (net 16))
 (segment (start 15.5 12.75) (end 37.4433 12.75) (width 2) (layer "F.Cu") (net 3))
 (segment (start 37.4433 25) (end 38.2981 25) (width 2) (layer "F.Cu") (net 3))
 (segment (start 38.2981 25) (end 38.5 25) (width 0.7998) (layer "F.Cu") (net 3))
 (via (at 37.4433 12.75) (size 0.6) (drill 0.3) (layers "F.Cu" "B.Cu") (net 3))
 (via (at 37.4433 25) (size 0.6) (drill 0.3) (layers "F.Cu" "B.Cu") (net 3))
 (segment (start 37.4433 25) (end 37.4433 12.75) (width 2) (layer "B.Cu") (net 3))
 (segment (start 46 33) (end 46 25) (width 0.76) (layer "F.Cu") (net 18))
 (segment (start 15.1 33) (end 46 33) (width 0.76) (layer "F.Cu") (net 18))
 (segment (start 46 33) (end 46 30) (width 0.76) (layer "F.Cu") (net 17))
 (segment (start 34.9 33) (end 46 33) (width 0.76) (layer "F.Cu") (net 17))
 (segment (start 8.5 30) (end 8.5 8.25) (width 0.25) (layer "F.Cu") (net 5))
 (segment (start 3.5 32) (end 3.5 30) (width 0.25) (layer "F.Cu") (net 5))
 (segment (start 3.5 30) (end 3.5 30) (width 0.25) (layer "F.Cu") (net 5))
 (segment (start 3.5 30) (end 3.5 30) (width 0.25) (layer "F.Cu") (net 5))
 (segment (start 3.5 30) (end 8.5 30) (width 0.25) (layer "F.Cu") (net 5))
 (segment (start 2.5 32) (end 3.5 32) (width 0.25) (layer "F.Cu") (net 5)))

